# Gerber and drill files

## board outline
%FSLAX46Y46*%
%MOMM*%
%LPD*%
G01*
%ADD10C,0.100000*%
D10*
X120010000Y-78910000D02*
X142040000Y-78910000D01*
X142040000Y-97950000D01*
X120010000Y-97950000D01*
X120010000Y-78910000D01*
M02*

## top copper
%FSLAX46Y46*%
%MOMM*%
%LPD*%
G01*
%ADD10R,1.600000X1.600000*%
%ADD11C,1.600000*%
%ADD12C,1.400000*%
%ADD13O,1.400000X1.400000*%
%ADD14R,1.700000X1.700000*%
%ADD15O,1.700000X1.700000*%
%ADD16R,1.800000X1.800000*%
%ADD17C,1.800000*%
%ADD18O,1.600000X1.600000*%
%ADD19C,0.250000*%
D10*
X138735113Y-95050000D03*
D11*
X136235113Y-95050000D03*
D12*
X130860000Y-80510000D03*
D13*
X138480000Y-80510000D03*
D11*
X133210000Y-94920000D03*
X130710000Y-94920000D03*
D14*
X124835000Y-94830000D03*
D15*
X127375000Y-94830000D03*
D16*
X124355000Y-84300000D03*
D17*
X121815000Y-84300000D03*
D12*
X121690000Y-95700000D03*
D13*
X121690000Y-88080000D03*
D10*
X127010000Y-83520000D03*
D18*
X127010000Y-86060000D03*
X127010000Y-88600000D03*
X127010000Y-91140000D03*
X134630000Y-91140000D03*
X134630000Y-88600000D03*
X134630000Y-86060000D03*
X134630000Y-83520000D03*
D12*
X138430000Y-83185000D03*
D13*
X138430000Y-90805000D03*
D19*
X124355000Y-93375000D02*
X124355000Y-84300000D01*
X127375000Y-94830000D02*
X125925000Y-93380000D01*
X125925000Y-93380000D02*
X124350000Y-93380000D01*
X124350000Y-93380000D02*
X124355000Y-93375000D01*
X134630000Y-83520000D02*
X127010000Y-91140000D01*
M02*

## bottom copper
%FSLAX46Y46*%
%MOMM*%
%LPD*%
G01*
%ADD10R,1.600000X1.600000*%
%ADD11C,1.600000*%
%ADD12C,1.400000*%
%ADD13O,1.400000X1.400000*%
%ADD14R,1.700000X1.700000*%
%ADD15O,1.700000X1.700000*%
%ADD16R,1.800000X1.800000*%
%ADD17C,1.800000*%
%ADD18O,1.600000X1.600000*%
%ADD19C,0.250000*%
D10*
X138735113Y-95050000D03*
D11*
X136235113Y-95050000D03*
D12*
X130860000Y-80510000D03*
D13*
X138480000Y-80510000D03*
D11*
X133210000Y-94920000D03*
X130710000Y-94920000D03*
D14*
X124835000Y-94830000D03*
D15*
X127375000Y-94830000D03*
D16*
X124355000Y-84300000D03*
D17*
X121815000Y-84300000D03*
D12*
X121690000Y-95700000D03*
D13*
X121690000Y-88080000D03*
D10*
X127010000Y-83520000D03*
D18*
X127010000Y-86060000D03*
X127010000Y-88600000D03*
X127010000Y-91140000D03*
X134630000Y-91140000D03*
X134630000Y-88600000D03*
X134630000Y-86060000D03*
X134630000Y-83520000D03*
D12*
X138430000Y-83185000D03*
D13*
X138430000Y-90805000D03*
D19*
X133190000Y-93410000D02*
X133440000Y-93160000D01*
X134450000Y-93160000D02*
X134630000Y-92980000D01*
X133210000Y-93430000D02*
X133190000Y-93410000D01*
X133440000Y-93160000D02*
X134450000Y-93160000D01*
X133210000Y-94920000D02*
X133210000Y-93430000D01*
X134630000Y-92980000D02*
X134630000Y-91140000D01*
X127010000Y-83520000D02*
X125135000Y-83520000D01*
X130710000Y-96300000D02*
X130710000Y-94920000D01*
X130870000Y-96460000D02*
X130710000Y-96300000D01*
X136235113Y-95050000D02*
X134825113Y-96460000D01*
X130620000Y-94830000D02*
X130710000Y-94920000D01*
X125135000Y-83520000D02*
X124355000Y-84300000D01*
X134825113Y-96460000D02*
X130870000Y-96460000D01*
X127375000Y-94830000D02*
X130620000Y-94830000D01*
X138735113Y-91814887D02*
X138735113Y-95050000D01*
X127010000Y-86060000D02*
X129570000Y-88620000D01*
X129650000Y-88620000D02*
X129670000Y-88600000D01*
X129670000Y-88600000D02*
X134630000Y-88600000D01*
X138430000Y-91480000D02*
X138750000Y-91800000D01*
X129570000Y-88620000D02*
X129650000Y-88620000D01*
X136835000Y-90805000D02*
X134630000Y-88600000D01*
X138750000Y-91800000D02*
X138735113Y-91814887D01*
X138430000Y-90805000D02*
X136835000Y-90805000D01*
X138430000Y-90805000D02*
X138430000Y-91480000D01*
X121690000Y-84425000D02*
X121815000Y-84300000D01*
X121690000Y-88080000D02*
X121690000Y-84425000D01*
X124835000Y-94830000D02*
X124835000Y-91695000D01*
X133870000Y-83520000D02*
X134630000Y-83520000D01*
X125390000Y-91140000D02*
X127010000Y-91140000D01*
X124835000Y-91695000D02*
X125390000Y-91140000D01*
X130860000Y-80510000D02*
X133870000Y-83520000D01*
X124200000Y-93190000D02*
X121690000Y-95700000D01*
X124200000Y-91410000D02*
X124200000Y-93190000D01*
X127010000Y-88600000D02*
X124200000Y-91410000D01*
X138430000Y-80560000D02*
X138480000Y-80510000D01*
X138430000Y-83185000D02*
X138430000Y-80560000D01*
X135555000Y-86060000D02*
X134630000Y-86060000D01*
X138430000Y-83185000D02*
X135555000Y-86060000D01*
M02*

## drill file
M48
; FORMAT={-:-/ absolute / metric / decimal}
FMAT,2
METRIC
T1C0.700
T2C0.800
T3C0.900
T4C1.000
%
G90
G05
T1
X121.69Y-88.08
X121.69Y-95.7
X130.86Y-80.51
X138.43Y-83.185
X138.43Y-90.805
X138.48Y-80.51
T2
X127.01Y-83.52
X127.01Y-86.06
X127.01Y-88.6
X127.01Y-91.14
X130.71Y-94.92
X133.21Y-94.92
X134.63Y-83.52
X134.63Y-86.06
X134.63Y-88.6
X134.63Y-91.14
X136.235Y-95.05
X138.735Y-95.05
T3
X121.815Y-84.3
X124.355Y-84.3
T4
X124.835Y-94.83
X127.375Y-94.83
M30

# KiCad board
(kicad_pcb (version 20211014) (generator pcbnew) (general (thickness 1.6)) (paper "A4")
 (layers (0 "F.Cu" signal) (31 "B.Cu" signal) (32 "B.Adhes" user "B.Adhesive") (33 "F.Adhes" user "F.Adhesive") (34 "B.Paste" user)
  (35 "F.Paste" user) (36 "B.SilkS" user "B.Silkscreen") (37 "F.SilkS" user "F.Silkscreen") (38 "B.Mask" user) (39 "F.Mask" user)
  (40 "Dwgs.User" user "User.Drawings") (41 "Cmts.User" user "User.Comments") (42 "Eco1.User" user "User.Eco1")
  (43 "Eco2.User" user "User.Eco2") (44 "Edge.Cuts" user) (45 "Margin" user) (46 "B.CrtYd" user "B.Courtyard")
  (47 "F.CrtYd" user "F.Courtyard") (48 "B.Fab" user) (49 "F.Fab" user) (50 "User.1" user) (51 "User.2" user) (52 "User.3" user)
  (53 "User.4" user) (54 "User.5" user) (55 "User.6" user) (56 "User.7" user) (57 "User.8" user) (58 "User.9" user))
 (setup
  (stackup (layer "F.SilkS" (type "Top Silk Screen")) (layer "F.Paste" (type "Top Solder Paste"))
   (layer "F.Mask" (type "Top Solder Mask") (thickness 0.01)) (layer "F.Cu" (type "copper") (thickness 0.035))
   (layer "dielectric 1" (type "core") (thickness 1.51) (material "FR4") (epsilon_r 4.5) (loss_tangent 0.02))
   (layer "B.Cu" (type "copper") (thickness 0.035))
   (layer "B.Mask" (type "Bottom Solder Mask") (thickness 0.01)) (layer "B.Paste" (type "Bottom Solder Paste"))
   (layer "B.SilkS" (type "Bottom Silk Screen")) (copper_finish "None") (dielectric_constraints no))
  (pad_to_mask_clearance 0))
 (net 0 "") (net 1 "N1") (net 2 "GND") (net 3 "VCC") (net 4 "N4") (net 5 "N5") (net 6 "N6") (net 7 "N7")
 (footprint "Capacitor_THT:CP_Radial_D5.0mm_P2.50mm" (layer "F.Cu") (at 138.735113 95.05 180)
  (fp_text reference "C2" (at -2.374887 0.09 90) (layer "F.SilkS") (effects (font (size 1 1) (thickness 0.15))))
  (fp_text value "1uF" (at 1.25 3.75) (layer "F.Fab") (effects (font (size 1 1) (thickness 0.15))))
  (pad "1" thru_hole rect (at 0 0 180) (size 1.6 1.6) (drill 0.8) (layers *.Cu *.Mask) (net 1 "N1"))
  (pad "2" thru_hole circle (at 2.5 0 180) (size 1.6 1.6) (drill 0.8) (layers *.Cu *.Mask) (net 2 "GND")))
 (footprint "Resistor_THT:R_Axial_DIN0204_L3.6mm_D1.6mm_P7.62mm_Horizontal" (layer "F.Cu") (at 130.86 80.51)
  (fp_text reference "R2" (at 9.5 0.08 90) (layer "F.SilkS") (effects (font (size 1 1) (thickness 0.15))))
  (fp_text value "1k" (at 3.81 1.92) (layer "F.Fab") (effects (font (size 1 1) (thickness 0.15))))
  (pad "1" thru_hole circle (at 0 0) (size 1.4 1.4) (drill 0.7) (layers *.Cu *.Mask) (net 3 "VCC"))
  (pad "2" thru_hole oval (at 7.62 0) (size 1.4 1.4) (drill 0.7) (layers *.Cu *.Mask) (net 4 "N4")))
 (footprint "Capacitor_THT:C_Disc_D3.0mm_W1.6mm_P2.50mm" (layer "F.Cu") (at 133.21 94.92 180)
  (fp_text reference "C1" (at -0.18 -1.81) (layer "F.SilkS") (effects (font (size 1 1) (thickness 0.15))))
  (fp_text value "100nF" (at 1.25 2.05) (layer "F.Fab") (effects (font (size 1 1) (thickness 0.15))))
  (pad "1" thru_hole circle (at 0 0 180) (size 1.6 1.6) (drill 0.8) (layers *.Cu *.Mask) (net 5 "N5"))
  (pad "2" thru_hole circle (at 2.5 0 180) (size 1.6 1.6) (drill 0.8) (layers *.Cu *.Mask) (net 2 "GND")))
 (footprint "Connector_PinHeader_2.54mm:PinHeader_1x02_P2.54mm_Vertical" (layer "F.Cu") (at 124.835 94.83 90)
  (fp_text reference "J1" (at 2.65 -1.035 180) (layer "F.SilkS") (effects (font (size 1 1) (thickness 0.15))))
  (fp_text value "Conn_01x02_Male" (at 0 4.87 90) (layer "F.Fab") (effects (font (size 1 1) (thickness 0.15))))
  (pad "1" thru_hole rect (at 0 0 90) (size 1.7 1.7) (drill 1) (layers *.Cu *.Mask) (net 3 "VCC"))
  (pad "2" thru_hole oval (at 0 2.54 90) (size 1.7 1.7) (drill 1) (layers *.Cu *.Mask) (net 2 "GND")))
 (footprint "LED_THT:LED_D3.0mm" (layer "F.Cu") (at 124.355 84.3 180)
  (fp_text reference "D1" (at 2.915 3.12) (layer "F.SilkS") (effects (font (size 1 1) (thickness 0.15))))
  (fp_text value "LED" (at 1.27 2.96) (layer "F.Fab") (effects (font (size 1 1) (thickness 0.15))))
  (pad "1" thru_hole rect (at 0 0 180) (size 1.8 1.8) (drill 0.9) (layers *.Cu *.Mask) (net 2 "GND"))
  (pad "2" thru_hole circle (at 2.54 0 180) (size 1.8 1.8) (drill 0.9) (layers *.Cu *.Mask) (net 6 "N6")))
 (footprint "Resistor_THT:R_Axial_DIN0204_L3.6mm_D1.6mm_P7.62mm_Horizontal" (layer "F.Cu") (at 121.69 95.7 90)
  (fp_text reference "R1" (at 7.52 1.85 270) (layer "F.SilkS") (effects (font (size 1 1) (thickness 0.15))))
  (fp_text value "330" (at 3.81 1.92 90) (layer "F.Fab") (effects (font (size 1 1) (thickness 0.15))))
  (pad "1" thru_hole circle (at 0 0 90) (size 1.4 1.4) (drill 0.7) (layers *.Cu *.Mask) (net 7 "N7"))
  (pad "2" thru_hole oval (at 7.62 0 90) (size 1.4 1.4) (drill 0.7) (layers *.Cu *.Mask) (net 6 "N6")))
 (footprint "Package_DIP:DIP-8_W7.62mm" (layer "F.Cu") (at 127.01 83.52)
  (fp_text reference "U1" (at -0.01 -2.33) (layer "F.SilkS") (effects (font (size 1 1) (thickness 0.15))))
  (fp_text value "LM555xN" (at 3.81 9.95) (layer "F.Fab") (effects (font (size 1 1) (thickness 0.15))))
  (pad "1" thru_hole rect (at 0 0) (size 1.6 1.6) (drill 0.8) (layers *.Cu *.Mask) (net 2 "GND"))
  (pad "2" thru_hole oval (at 0 2.54) (size 1.6 1.6) (drill 0.8) (layers *.Cu *.Mask) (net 1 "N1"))
  (pad "3" thru_hole oval (at 0 5.08) (size 1.6 1.6) (drill 0.8) (layers *.Cu *.Mask) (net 7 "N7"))
  (pad "4" thru_hole oval (at 0 7.62) (size 1.6 1.6) (drill 0.8) (layers *.Cu *.Mask) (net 3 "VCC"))
  (pad "5" thru_hole oval (at 7.62 7.62) (size 1.6 1.6) (drill 0.8) (layers *.Cu *.Mask) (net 5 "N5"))
  (pad "6" thru_hole oval (at 7.62 5.08) (size 1.6 1.6) (drill 0.8) (layers *.Cu *.Mask) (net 1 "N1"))
  (pad "7" thru_hole oval (at 7.62 2.54) (size 1.6 1.6) (drill 0.8) (layers *.Cu *.Mask) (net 4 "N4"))
  (pad "8" thru_hole oval (at 7.62 0) (size 1.6 1.6) (drill 0.8) (layers *.Cu *.Mask) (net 3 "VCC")))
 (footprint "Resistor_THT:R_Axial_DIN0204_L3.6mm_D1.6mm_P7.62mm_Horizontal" (layer "F.Cu") (at 138.43 83.185 -90)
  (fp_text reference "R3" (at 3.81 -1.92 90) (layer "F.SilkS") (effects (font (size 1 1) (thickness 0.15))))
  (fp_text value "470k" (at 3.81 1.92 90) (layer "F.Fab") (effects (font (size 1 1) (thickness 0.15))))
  (pad "1" thru_hole circle (at 0 0 270) (size 1.4 1.4) (drill 0.7) (layers *.Cu *.Mask) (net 4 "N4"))
  (pad "2" thru_hole oval (at 7.62 0 270) (size 1.4 1.4) (drill 0.7) (layers *.Cu *.Mask) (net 1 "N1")))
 (gr_rect (start 120.01 78.91) (end 142.04 97.95) (layer "Edge.Cuts") (width 0.1) (fill none))
 (segment (start 133.19 93.41) (end 133.44 93.16) (width 0.25) (layer "B.Cu") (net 5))
 (segment (start 134.45 93.16) (end 134.63 92.98) (width 0.25) (layer "B.Cu") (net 5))
 (segment (start 133.21 93.43) (end 133.19 93.41) (width 0.25) (layer "B.Cu") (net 5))
 (segment (start 133.44 93.16) (end 134.45 93.16) (width 0.25) (layer "B.Cu") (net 5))
 (segment (start 133.21 94.92) (end 133.21 93.43) (width 0.25) (layer "B.Cu") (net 5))
 (segment (start 134.63 92.98) (end 134.63 91.14) (width 0.25) (layer "B.Cu") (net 5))
 (segment (start 124.355 93.375) (end 124.355 84.3) (width 0.25) (layer "F.Cu") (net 2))
 (segment (start 127.375 94.83) (end 125.925 93.38) (width 0.25) (layer "F.Cu") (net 2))
 (segment (start 125.925 93.38) (end 124.35 93.38) (width 0.25) (layer "F.Cu") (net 2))
 (segment (start 124.35 93.38) (end 124.355 93.375) (width 0.25) (layer "F.Cu") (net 2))
 (segment (start 127.01 83.52) (end 125.135 83.52) (width 0.25) (layer "B.Cu") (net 2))
 (segment (start 130.71 96.3) (end 130.71 94.92) (width 0.25) (layer "B.Cu") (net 2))
 (segment (start 130.87 96.46) (end 130.71 96.3) (width 0.25) (layer "B.Cu") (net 2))
 (segment (start 136.235113 95.05) (end 134.825113 96.46) (width 0.25) (layer "B.Cu") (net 2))
 (segment (start 130.62 94.83) (end 130.71 94.92) (width 0.25) (layer "B.Cu") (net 2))
 (segment (start 125.135 83.52) (end 124.355 84.3) (width 0.25) (layer "B.Cu") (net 2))
 (segment (start 134.825113 96.46) (end 130.87 96.46) (width 0.25) (layer "B.Cu") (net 2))
 (segment (start 127.375 94.83) (end 130.62 94.83) (width 0.25) (layer "B.Cu") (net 2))
 (segment (start 138.735113 91.814887) (end 138.735113 95.05) (width 0.25) (layer "B.Cu") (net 1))
 (segment (start 127.01 86.06) (end 129.57 88.62) (width 0.25) (layer "B.Cu") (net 1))
 (segment (start 129.65 88.62) (end 129.67 88.6) (width 0.25) (layer "B.Cu") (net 1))
 (segment (start 129.67 88.6) (end 134.63 88.6) (width 0.25) (layer "B.Cu") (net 1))
 (segment (start 138.43 91.48) (end 138.75 91.8) (width 0.25) (layer "B.Cu") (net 1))
 (segment (start 129.57 88.62) (end 129.65 88.62) (width 0.25) (layer "B.Cu") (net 1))
 (segment (start 136.835 90.805) (end 134.63 88.6) (width 0.25) (layer "B.Cu") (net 1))
 (segment (start 138.75 91.8) (end 138.735113 91.814887) (width 0.25) (layer "B.Cu") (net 1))
 (segment (start 138.43 90.805) (end 136.835 90.805) (width 0.25) (layer "B.Cu") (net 1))
 (segment (start 138.43 90.805) (end 138.43 91.48) (width 0.25) (layer "B.Cu") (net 1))
 (segment (start 121.69 84.425) (end 121.815 84.3) (width 0.25) (layer "B.Cu") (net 6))
 (segment (start 121.69 88.08) (end 121.69 84.425) (width 0.25) (layer "B.Cu") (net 6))
 (segment (start 134.63 83.52) (end 127.01 91.14) (width 0.25) (layer "F.Cu") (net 3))
 (segment (start 124.835 94.83) (end 124.835 91.695) (width 0.25) (layer "B.Cu") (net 3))
 (segment (start 133.87 83.52) (end 134.63 83.52) (width 0.25) (layer "B.Cu") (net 3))
 (segment (start 125.39 91.14) (end 127.01 91.14) (width 0.25) (layer "B.Cu") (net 3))
 (segment (start 124.835 91.695) (end 125.39 91.14) (width 0.25) (layer "B.Cu") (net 3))
 (segment (start 130.86 80.51) (end 133.87 83.52) (width 0.25) (layer "B.Cu") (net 3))
 (segment (start 124.2 93.19) (end 121.69 95.7) (width 0.25) (layer "B.Cu") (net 7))
 (segment (start 124.2 91.41) (end 124.2 93.19) (width 0.25) (layer "B.Cu") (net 7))
 (segment (start 127.01 88.6) (end 124.2 91.41) (width 0.25) (layer "B.Cu") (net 7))
 (segment (start 138.43 80.56) (end 138.48 80.51) (width 0.25) (layer "B.Cu") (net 4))
 (segment (start 138.43 83.185) (end 138.43 80.56) (width 0.25) (layer "B.Cu") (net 4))
 (segment (start 135.555 86.06) (end 134.63 86.06) (width 0.25) (layer "B.Cu") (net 4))
 (segment (start 138.43 83.185) (end 135.555 86.06) (width 0.25) (layer "B.Cu") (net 4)))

